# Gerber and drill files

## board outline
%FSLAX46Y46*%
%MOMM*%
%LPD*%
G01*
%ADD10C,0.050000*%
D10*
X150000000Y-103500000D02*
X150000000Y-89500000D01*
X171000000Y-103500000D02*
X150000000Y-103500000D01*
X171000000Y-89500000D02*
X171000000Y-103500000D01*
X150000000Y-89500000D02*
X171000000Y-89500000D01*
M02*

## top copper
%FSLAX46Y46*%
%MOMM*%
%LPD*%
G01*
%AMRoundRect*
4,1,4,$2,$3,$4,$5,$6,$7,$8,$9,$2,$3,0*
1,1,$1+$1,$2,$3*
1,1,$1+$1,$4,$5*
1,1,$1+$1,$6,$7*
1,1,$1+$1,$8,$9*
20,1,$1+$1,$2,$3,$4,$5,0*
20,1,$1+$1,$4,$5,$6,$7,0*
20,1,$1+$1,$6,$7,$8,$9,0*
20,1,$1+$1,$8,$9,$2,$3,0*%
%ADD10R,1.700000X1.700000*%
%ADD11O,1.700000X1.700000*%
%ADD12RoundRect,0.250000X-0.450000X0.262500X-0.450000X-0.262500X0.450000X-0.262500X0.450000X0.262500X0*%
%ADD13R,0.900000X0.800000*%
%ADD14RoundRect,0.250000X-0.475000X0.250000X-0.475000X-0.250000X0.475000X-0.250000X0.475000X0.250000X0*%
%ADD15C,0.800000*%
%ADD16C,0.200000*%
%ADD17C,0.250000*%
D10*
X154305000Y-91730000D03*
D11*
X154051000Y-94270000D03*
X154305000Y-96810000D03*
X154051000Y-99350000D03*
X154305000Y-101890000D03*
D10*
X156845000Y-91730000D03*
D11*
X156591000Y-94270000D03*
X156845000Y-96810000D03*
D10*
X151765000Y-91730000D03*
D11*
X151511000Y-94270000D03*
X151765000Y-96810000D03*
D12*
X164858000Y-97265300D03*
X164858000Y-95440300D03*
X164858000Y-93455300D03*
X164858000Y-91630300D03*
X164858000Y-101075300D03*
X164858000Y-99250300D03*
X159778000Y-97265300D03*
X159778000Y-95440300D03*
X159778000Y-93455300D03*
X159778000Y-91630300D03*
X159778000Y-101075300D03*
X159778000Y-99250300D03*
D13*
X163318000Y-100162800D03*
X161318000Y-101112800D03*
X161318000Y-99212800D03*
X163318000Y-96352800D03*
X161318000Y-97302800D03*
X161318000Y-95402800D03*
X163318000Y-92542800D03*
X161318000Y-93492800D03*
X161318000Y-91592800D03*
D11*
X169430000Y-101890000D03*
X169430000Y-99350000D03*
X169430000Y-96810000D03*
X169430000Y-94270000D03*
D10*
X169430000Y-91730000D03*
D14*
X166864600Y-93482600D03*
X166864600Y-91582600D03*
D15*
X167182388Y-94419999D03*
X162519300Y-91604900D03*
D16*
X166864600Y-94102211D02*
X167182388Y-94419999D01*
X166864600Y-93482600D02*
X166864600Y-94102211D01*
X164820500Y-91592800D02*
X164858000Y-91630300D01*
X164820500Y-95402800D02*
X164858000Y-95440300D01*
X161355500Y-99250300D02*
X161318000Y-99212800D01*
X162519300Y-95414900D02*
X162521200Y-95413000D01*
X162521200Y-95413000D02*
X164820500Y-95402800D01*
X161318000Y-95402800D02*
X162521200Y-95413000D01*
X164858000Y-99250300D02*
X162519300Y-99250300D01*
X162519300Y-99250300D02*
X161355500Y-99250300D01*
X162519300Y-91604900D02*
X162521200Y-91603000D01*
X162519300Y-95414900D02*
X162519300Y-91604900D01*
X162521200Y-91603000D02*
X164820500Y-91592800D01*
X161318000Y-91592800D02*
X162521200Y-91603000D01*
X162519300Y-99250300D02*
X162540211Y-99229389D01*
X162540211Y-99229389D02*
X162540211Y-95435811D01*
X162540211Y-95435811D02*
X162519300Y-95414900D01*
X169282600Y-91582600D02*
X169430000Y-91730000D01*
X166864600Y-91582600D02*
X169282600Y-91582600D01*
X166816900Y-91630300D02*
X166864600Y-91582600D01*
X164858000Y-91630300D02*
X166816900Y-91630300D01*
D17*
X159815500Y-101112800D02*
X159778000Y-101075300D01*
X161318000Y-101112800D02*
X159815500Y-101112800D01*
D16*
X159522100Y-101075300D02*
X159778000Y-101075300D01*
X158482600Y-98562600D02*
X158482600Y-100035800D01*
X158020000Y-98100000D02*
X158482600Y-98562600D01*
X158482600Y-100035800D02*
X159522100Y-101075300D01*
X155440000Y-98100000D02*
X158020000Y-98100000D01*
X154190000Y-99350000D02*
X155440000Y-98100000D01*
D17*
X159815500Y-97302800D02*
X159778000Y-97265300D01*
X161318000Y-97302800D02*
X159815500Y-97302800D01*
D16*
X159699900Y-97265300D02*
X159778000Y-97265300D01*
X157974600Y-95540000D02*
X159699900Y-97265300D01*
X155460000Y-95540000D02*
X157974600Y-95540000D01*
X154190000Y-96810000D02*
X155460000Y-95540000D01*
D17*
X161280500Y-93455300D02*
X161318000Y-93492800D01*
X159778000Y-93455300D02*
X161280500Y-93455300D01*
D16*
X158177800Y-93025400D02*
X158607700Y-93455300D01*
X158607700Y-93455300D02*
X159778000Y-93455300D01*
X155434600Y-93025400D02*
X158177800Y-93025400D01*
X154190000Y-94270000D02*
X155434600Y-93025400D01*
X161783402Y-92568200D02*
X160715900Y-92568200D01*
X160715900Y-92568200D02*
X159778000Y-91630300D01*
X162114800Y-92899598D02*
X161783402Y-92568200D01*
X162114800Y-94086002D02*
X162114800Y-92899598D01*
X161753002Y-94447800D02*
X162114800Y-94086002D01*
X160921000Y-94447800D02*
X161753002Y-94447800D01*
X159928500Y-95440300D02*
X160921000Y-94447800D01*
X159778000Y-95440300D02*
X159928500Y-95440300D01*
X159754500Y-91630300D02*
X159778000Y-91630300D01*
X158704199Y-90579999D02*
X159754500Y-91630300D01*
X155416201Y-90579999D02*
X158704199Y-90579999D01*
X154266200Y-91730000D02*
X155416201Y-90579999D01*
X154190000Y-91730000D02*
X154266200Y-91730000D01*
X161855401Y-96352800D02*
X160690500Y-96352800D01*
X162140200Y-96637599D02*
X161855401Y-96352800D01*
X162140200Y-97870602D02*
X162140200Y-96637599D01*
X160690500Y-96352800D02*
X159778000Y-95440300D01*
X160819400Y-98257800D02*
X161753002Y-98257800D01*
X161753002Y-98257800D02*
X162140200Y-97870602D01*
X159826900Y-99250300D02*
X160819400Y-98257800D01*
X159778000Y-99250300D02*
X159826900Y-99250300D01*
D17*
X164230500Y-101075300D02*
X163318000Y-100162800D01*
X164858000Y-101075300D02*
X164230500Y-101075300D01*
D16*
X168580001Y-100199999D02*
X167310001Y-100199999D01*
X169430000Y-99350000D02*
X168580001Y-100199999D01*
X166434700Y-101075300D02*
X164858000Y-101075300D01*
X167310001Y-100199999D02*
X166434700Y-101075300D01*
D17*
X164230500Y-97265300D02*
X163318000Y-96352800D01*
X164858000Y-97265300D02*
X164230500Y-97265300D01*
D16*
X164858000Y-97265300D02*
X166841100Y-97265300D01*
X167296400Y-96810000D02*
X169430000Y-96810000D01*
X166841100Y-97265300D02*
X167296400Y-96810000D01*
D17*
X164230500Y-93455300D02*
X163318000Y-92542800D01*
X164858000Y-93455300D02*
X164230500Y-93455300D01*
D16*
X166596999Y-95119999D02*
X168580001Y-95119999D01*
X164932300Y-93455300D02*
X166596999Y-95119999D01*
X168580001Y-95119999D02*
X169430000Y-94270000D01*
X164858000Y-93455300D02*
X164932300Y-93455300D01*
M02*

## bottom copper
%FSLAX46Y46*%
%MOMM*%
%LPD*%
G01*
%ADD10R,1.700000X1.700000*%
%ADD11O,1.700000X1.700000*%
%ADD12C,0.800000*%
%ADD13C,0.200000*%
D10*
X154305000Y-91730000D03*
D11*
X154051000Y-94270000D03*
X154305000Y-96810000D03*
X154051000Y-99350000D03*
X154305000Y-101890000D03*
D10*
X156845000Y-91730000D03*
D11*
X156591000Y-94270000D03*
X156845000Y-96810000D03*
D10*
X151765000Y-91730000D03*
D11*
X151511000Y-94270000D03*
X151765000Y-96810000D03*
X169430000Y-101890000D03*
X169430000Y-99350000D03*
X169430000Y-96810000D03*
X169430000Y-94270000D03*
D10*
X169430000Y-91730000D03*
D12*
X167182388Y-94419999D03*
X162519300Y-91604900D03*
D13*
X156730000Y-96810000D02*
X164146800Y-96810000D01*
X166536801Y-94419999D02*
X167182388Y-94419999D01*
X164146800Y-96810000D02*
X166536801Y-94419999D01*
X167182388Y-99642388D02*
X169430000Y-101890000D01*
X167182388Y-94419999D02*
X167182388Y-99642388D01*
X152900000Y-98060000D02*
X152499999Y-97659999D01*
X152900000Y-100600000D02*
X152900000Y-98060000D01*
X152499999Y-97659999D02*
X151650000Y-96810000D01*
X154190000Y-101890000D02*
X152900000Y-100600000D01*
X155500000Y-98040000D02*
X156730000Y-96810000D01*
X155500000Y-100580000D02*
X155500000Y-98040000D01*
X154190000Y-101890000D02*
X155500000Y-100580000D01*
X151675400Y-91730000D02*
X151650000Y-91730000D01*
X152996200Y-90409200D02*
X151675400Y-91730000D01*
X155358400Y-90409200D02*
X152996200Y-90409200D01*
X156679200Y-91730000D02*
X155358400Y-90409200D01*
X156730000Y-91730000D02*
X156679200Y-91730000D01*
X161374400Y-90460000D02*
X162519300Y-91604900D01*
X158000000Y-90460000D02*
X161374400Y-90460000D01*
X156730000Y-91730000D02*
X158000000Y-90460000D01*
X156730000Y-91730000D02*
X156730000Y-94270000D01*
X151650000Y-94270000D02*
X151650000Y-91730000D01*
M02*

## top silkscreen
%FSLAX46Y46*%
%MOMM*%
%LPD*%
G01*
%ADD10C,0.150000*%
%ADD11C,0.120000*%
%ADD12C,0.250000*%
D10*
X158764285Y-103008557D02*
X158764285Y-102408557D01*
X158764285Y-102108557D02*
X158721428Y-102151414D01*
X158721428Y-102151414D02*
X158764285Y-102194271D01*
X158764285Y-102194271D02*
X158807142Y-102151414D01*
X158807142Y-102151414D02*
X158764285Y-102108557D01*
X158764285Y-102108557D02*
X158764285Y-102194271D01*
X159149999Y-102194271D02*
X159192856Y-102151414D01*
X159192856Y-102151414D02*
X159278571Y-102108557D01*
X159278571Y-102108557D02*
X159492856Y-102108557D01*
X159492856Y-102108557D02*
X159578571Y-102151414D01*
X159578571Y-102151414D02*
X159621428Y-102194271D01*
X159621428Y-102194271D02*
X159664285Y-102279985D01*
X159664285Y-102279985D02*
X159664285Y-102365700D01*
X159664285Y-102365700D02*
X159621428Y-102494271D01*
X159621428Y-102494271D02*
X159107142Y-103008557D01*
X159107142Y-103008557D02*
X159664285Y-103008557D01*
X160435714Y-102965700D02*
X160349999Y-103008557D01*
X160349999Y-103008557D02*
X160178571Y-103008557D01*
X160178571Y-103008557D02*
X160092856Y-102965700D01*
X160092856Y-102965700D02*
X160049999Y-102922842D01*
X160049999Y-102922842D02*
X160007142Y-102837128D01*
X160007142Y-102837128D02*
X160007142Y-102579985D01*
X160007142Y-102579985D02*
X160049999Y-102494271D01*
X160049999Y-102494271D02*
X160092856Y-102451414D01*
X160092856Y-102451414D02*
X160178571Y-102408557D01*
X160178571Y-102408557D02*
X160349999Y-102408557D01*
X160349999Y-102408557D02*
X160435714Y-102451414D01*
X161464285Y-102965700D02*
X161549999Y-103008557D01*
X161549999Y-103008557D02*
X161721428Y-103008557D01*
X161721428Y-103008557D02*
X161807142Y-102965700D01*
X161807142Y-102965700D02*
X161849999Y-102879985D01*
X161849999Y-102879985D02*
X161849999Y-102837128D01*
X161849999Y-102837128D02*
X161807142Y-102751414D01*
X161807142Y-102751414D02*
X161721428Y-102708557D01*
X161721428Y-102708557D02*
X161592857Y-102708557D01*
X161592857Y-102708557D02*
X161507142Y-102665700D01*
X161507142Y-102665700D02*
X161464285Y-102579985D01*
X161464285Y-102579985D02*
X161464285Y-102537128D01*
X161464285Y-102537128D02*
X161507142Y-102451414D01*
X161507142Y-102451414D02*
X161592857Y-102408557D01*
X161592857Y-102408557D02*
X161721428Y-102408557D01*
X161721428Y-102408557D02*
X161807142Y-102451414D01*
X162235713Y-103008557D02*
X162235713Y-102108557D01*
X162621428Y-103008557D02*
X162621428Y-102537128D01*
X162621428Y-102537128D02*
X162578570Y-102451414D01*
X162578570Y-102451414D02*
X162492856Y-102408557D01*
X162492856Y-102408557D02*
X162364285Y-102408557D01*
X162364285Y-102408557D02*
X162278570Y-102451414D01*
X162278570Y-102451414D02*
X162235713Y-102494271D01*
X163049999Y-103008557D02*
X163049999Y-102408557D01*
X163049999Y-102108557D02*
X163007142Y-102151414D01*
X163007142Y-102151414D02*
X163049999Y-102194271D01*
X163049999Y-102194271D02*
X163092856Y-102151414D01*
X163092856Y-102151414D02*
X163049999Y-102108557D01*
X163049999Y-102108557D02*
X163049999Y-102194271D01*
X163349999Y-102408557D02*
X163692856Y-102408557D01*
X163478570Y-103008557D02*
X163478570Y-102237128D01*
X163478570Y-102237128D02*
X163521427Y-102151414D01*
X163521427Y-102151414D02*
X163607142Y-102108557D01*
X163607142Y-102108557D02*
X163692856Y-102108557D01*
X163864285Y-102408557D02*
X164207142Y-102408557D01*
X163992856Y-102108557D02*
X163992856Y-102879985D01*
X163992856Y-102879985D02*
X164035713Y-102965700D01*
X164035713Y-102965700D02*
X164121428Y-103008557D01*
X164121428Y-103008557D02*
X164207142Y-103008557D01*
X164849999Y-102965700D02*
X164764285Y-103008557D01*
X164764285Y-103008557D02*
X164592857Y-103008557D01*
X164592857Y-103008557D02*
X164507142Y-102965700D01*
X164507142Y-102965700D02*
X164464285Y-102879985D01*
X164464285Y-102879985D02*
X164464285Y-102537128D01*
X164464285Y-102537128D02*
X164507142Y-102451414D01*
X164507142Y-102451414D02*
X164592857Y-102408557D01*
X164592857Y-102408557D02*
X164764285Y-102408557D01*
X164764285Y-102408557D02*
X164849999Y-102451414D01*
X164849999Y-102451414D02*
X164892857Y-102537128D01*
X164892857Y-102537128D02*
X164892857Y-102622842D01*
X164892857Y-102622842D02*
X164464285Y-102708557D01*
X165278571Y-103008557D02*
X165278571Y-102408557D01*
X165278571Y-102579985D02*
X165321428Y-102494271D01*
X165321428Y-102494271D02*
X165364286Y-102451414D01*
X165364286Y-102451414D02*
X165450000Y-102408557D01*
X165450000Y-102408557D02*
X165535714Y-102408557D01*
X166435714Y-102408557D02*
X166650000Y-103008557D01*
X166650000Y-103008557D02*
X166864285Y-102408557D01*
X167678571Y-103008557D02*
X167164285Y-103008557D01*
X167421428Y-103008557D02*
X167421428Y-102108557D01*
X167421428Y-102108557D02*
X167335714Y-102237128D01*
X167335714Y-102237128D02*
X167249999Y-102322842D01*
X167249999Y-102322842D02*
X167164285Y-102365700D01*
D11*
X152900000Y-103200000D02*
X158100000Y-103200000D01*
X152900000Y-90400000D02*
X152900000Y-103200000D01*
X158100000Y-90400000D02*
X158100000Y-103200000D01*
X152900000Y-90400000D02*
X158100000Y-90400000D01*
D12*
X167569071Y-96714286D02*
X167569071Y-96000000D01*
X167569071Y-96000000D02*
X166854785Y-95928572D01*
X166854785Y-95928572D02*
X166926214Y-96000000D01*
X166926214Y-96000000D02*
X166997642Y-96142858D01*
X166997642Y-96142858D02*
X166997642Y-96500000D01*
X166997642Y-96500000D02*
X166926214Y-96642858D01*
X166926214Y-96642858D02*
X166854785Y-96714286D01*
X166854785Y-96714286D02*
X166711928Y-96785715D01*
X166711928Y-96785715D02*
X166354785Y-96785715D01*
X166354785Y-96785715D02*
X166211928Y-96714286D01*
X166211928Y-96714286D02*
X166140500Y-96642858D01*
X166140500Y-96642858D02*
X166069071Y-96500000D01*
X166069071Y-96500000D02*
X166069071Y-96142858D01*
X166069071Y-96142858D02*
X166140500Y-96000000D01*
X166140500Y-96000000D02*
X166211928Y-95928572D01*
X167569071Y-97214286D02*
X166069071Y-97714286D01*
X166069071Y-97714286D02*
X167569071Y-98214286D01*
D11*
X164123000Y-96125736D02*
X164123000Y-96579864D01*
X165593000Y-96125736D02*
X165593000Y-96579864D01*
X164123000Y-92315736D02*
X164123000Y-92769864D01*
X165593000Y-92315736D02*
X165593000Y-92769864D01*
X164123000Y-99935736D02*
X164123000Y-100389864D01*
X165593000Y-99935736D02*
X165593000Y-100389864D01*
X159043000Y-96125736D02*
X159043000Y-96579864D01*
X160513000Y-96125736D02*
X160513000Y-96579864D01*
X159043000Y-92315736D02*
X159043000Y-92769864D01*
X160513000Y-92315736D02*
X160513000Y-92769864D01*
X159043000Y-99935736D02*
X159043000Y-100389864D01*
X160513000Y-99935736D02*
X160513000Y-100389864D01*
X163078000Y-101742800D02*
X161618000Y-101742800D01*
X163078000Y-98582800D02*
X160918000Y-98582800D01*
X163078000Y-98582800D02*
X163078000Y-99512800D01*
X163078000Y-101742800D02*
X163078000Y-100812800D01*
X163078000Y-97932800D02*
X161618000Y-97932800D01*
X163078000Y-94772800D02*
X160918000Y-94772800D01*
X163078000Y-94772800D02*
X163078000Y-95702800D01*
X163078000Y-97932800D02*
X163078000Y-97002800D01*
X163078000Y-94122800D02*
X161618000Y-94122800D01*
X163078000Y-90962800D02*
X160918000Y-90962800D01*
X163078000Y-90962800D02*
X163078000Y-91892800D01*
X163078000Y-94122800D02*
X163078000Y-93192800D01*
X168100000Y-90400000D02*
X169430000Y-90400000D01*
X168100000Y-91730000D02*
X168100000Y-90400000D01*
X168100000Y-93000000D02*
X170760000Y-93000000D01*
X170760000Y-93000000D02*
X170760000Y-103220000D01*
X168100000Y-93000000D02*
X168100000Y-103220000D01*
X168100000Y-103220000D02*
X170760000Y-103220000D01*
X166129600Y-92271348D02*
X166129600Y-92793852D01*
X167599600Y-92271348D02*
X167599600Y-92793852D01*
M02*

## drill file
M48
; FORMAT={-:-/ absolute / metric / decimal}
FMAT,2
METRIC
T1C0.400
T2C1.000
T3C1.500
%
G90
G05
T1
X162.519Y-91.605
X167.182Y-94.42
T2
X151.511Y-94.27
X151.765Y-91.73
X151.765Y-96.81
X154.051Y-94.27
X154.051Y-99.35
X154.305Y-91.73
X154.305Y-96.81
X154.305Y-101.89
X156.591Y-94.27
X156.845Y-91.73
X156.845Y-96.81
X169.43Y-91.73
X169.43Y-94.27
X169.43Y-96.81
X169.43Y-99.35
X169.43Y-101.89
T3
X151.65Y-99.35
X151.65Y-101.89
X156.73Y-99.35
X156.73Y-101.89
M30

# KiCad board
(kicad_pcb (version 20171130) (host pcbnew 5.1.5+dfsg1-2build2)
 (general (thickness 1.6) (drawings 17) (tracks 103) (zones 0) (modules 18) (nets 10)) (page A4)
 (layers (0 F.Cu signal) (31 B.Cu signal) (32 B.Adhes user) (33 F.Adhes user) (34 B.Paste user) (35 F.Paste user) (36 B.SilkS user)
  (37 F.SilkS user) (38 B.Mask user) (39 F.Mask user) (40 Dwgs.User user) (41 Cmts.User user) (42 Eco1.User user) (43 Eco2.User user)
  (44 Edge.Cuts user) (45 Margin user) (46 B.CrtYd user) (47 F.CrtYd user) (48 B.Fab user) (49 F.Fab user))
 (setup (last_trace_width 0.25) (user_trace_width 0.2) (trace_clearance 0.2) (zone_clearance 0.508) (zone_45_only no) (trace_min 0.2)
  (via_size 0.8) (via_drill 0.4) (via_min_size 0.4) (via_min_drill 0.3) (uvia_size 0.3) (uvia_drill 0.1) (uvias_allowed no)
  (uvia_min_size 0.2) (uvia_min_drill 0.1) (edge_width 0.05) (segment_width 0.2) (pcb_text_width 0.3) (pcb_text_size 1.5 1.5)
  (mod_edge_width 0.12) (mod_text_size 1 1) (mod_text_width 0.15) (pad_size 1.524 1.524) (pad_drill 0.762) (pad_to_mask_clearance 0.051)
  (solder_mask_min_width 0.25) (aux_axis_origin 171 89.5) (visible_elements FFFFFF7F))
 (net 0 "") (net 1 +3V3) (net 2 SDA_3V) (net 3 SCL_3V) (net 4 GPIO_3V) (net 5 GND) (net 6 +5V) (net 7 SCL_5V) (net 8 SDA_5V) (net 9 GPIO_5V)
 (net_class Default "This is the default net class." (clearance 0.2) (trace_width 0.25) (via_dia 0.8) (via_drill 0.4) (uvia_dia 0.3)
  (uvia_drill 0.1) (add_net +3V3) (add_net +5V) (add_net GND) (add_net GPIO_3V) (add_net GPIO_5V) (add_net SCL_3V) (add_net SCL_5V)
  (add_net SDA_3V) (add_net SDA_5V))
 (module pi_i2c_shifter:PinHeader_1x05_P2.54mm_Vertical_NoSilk (layer F.Cu) (at 154.19 91.73)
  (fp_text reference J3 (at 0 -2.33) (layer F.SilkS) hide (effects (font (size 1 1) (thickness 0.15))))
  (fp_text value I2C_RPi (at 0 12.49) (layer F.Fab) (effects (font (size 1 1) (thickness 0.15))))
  (pad 1 thru_hole rect (at 0.115 0) (size 1.7 1.7) (drill 1) (layers *.Cu *.Mask) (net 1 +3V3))
  (pad 2 thru_hole oval (at -0.139 2.54) (size 1.7 1.7) (drill 1) (layers *.Cu *.Mask) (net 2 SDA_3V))
  (pad 3 thru_hole oval (at 0.115 5.08) (size 1.7 1.7) (drill 1) (layers *.Cu *.Mask) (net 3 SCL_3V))
  (pad 4 thru_hole oval (at -0.139 7.62) (size 1.7 1.7) (drill 1) (layers *.Cu *.Mask) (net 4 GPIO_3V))
  (pad 5 thru_hole oval (at 0.115 10.16) (size 1.7 1.7) (drill 1) (layers *.Cu *.Mask) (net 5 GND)))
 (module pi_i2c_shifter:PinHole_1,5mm (layer F.Cu) (at 151.65 99.35)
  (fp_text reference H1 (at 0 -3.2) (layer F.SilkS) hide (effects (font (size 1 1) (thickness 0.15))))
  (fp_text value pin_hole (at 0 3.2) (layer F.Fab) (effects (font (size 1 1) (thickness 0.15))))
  (pad "" np_thru_hole circle (at 0 0) (size 1.5 1.5) (drill 1.5) (layers *.Cu *.Mask)))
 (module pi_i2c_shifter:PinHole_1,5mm (layer F.Cu) (at 151.65 101.89)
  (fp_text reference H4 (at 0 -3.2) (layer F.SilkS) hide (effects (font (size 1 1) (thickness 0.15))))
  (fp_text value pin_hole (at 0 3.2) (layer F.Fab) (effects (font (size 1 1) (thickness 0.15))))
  (pad "" np_thru_hole circle (at 0 0) (size 1.5 1.5) (drill 1.5) (layers *.Cu *.Mask)))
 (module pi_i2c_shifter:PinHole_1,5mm (layer F.Cu) (at 156.73 99.35)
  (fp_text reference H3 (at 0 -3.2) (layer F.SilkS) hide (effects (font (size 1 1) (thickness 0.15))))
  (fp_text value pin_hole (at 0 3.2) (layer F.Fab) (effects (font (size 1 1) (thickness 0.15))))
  (pad "" np_thru_hole circle (at 0 0) (size 1.5 1.5) (drill 1.5) (layers *.Cu *.Mask)))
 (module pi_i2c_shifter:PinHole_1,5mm (layer F.Cu) (at 156.73 101.89)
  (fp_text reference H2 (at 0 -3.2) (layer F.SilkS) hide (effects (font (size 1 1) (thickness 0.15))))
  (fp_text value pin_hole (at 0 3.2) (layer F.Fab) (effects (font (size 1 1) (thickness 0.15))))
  (pad "" np_thru_hole circle (at 0 0) (size 1.5 1.5) (drill 1.5) (layers *.Cu *.Mask)))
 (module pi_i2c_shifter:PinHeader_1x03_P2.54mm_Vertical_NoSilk (layer F.Cu) (at 156.73 91.73)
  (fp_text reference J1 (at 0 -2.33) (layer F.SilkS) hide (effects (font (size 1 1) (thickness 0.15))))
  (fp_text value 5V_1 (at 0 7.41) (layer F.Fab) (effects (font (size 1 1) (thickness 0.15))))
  (pad 1 thru_hole rect (at 0.115 0) (size 1.7 1.7) (drill 1) (layers *.Cu *.Mask) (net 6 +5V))
  (pad 2 thru_hole oval (at -0.139 2.54) (size 1.7 1.7) (drill 1) (layers *.Cu *.Mask) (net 6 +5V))
  (pad 3 thru_hole oval (at 0.115 5.08) (size 1.7 1.7) (drill 1) (layers *.Cu *.Mask) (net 5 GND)))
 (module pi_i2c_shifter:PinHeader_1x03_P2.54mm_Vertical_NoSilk (layer F.Cu) (at 151.65 91.73)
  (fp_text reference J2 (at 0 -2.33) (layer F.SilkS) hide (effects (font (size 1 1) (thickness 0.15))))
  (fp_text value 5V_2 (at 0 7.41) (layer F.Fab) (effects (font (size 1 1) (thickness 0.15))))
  (pad 1 thru_hole rect (at 0.115 0) (size 1.7 1.7) (drill 1) (layers *.Cu *.Mask) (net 6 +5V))
  (pad 2 thru_hole oval (at -0.139 2.54) (size 1.7 1.7) (drill 1) (layers *.Cu *.Mask) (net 6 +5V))
  (pad 3 thru_hole oval (at 0.115 5.08) (size 1.7 1.7) (drill 1) (layers *.Cu *.Mask) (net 5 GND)))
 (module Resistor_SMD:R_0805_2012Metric (layer F.Cu) (at 164.858 96.3528 270)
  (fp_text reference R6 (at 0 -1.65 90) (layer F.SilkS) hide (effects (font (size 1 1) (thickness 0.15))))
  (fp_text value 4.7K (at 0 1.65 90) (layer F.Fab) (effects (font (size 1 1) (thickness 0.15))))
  (fp_line (start -0.227064 0.735) (end 0.227064 0.735) (layer F.SilkS) (width 0.12))
  (fp_line (start -0.227064 -0.735) (end 0.227064 -0.735) (layer F.SilkS) (width 0.12))
  (pad 2 smd roundrect (at 0.9125 0 270) (size 1.025 1.4) (layers F.Cu F.Paste F.Mask) (roundrect_rratio 0.243902) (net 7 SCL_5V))
  (pad 1 smd roundrect (at -0.9125 0 270) (size 1.025 1.4) (layers F.Cu F.Paste F.Mask) (roundrect_rratio 0.243902) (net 6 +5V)))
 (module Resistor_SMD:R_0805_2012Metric (layer F.Cu) (at 164.858 92.5428 270)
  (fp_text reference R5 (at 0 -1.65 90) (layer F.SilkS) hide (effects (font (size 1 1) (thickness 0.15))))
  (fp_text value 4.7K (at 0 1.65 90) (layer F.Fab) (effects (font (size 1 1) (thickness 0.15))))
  (fp_line (start -0.227064 0.735) (end 0.227064 0.735) (layer F.SilkS) (width 0.12))
  (fp_line (start -0.227064 -0.735) (end 0.227064 -0.735) (layer F.SilkS) (width 0.12))
  (pad 2 smd roundrect (at 0.9125 0 270) (size 1.025 1.4) (layers F.Cu F.Paste F.Mask) (roundrect_rratio 0.243902) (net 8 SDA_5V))
  (pad 1 smd roundrect (at -0.9125 0 270) (size 1.025 1.4) (layers F.Cu F.Paste F.Mask) (roundrect_rratio 0.243902) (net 6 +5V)))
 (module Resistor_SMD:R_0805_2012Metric (layer F.Cu) (at 164.858 100.1628 270)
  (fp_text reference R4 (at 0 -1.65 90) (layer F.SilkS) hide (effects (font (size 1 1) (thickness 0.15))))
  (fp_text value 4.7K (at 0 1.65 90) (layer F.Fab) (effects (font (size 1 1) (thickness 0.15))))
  (fp_line (start -0.227064 0.735) (end 0.227064 0.735) (layer F.SilkS) (width 0.12))
  (fp_line (start -0.227064 -0.735) (end 0.227064 -0.735) (layer F.SilkS) (width 0.12))
  (pad 2 smd roundrect (at 0.9125 0 270) (size 1.025 1.4) (layers F.Cu F.Paste F.Mask) (roundrect_rratio 0.243902) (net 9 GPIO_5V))
  (pad 1 smd roundrect (at -0.9125 0 270) (size 1.025 1.4) (layers F.Cu F.Paste F.Mask) (roundrect_rratio 0.243902) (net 6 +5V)))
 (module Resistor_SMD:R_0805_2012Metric (layer F.Cu) (at 159.778 96.3528 270)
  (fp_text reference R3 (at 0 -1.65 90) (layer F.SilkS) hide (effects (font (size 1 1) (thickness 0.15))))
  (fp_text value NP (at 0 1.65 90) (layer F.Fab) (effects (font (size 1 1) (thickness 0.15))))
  (fp_line (start -0.227064 0.735) (end 0.227064 0.735) (layer F.SilkS) (width 0.12))
  (fp_line (start -0.227064 -0.735) (end 0.227064 -0.735) (layer F.SilkS) (width 0.12))
  (pad 2 smd roundrect (at 0.9125 0 270) (size 1.025 1.4) (layers F.Cu F.Paste F.Mask) (roundrect_rratio 0.243902) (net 3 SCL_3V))
  (pad 1 smd roundrect (at -0.9125 0 270) (size 1.025 1.4) (layers F.Cu F.Paste F.Mask) (roundrect_rratio 0.243902) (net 1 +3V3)))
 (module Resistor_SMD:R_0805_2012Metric (layer F.Cu) (at 159.778 92.5428 270)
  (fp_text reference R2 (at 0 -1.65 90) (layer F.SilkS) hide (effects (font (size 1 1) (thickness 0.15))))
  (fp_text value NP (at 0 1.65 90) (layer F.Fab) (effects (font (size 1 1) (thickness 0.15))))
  (fp_line (start -0.227064 0.735) (end 0.227064 0.735) (layer F.SilkS) (width 0.12))
  (fp_line (start -0.227064 -0.735) (end 0.227064 -0.735) (layer F.SilkS) (width 0.12))
  (pad 2 smd roundrect (at 0.9125 0 270) (size 1.025 1.4) (layers F.Cu F.Paste F.Mask) (roundrect_rratio 0.243902) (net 2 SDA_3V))
  (pad 1 smd roundrect (at -0.9125 0 270) (size 1.025 1.4) (layers F.Cu F.Paste F.Mask) (roundrect_rratio 0.243902) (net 1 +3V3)))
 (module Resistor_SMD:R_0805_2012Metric (layer F.Cu) (at 159.778 100.1628 270)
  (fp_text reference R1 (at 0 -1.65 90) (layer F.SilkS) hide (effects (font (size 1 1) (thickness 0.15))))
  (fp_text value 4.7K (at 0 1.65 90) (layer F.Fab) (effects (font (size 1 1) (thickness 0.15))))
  (fp_line (start -0.227064 0.735) (end 0.227064 0.735) (layer F.SilkS) (width 0.12))
  (fp_line (start -0.227064 -0.735) (end 0.227064 -0.735) (layer F.SilkS) (width 0.12))
  (pad 2 smd roundrect (at 0.9125 0 270) (size 1.025 1.4) (layers F.Cu F.Paste F.Mask) (roundrect_rratio 0.243902) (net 4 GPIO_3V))
  (pad 1 smd roundrect (at -0.9125 0 270) (size 1.025 1.4) (layers F.Cu F.Paste F.Mask) (roundrect_rratio 0.243902) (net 1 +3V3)))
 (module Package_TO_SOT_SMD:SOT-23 (layer F.Cu) (at 162.318 100.1628)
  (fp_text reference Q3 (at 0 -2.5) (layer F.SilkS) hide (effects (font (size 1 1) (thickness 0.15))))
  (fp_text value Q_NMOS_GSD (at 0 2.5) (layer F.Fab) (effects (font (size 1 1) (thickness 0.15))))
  (fp_line (start 0.76 1.58) (end -0.7 1.58) (layer F.SilkS) (width 0.12))
  (fp_line (start 0.76 -1.58) (end -1.4 -1.58) (layer F.SilkS) (width 0.12))
  (fp_line (start 0.76 -1.58) (end 0.76 -0.65) (layer F.SilkS) (width 0.12))
  (fp_line (start 0.76 1.58) (end 0.76 0.65) (layer F.SilkS) (width 0.12))
  (pad 3 smd rect (at 1 0) (size 0.9 0.8) (layers F.Cu F.Paste F.Mask) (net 9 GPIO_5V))
  (pad 2 smd rect (at -1 0.95) (size 0.9 0.8) (layers F.Cu F.Paste F.Mask) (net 4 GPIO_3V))
  (pad 1 smd rect (at -1 -0.95) (size 0.9 0.8) (layers F.Cu F.Paste F.Mask) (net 6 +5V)))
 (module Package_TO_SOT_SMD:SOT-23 (layer F.Cu) (at 162.318 96.3528)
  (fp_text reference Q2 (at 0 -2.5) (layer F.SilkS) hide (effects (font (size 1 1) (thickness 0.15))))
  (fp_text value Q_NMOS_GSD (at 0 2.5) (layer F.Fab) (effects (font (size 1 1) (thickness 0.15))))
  (fp_line (start 0.76 1.58) (end -0.7 1.58) (layer F.SilkS) (width 0.12))
  (fp_line (start 0.76 -1.58) (end -1.4 -1.58) (layer F.SilkS) (width 0.12))
  (fp_line (start 0.76 -1.58) (end 0.76 -0.65) (layer F.SilkS) (width 0.12))
  (fp_line (start 0.76 1.58) (end 0.76 0.65) (layer F.SilkS) (width 0.12))
  (pad 3 smd rect (at 1 0) (size 0.9 0.8) (layers F.Cu F.Paste F.Mask) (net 7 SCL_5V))
  (pad 2 smd rect (at -1 0.95) (size 0.9 0.8) (layers F.Cu F.Paste F.Mask) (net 3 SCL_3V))
  (pad 1 smd rect (at -1 -0.95) (size 0.9 0.8) (layers F.Cu F.Paste F.Mask) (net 6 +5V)))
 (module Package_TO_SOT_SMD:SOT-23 (layer F.Cu) (at 162.318 92.5428)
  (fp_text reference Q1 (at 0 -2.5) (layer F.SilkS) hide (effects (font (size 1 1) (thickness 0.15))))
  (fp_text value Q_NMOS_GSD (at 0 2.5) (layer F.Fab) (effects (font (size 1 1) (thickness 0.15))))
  (fp_line (start 0.76 1.58) (end -0.7 1.58) (layer F.SilkS) (width 0.12))
  (fp_line (start 0.76 -1.58) (end -1.4 -1.58) (layer F.SilkS) (width 0.12))
  (fp_line (start 0.76 -1.58) (end 0.76 -0.65) (layer F.SilkS) (width 0.12))
  (fp_line (start 0.76 1.58) (end 0.76 0.65) (layer F.SilkS) (width 0.12))
  (pad 3 smd rect (at 1 0) (size 0.9 0.8) (layers F.Cu F.Paste F.Mask) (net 8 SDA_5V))
  (pad 2 smd rect (at -1 0.95) (size 0.9 0.8) (layers F.Cu F.Paste F.Mask) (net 2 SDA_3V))
  (pad 1 smd rect (at -1 -0.95) (size 0.9 0.8) (layers F.Cu F.Paste F.Mask) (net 6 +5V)))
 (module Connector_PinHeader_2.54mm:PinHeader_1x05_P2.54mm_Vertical (layer F.Cu) (at 169.43 91.73)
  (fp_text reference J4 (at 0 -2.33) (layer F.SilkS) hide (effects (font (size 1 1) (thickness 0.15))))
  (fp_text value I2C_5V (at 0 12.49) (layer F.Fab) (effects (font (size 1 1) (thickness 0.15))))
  (fp_line (start -1.33 -1.33) (end 0 -1.33) (layer F.SilkS) (width 0.12))
  (fp_line (start -1.33 0) (end -1.33 -1.33) (layer F.SilkS) (width 0.12))
  (fp_line (start -1.33 1.27) (end 1.33 1.27) (layer F.SilkS) (width 0.12))
  (fp_line (start 1.33 1.27) (end 1.33 11.49) (layer F.SilkS) (width 0.12))
  (fp_line (start -1.33 1.27) (end -1.33 11.49) (layer F.SilkS) (width 0.12))
  (fp_line (start -1.33 11.49) (end 1.33 11.49) (layer F.SilkS) (width 0.12))
  (pad 5 thru_hole oval (at 0 10.16) (size 1.7 1.7) (drill 1) (layers *.Cu *.Mask) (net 5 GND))
  (pad 4 thru_hole oval (at 0 7.62) (size 1.7 1.7) (drill 1) (layers *.Cu *.Mask) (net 9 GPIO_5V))
  (pad 3 thru_hole oval (at 0 5.08) (size 1.7 1.7) (drill 1) (layers *.Cu *.Mask) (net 7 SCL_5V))
  (pad 2 thru_hole oval (at 0 2.54) (size 1.7 1.7) (drill 1) (layers *.Cu *.Mask) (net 8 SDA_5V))
  (pad 1 thru_hole rect (at 0 0) (size 1.7 1.7) (drill 1) (layers *.Cu *.Mask) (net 6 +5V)))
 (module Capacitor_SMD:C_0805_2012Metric (layer F.Cu) (at 166.8646 92.5326 270)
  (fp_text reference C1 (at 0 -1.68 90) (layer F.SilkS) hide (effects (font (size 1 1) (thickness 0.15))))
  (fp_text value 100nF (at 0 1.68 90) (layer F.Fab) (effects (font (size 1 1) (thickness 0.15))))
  (fp_line (start -0.261252 0.735) (end 0.261252 0.735) (layer F.SilkS) (width 0.12))
  (fp_line (start -0.261252 -0.735) (end 0.261252 -0.735) (layer F.SilkS) (width 0.12))
  (pad 2 smd roundrect (at 0.95 0 270) (size 1 1.45) (layers F.Cu F.Paste F.Mask) (roundrect_rratio 0.25) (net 5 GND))
  (pad 1 smd roundrect (at -0.95 0 270) (size 1 1.45) (layers F.Cu F.Paste F.Mask) (roundrect_rratio 0.25) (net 6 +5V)))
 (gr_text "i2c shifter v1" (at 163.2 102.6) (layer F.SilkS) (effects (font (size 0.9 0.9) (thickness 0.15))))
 (gr_line (start 152.9 103.2) (end 158.1 103.2) (layer F.SilkS) (width 0.12))
 (gr_line (start 152.9 90.4) (end 152.9 103.2) (layer F.SilkS) (width 0.12))
 (gr_line (start 158.1 90.4) (end 158.1 103.2) (layer F.SilkS) (width 0.12))
 (gr_line (start 152.9 90.4) (end 158.1 90.4) (layer F.SilkS) (width 0.12))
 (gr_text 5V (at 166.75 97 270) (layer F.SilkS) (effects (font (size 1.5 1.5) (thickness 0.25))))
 (gr_line (start 150 103.5) (end 150 89.5) (layer Edge.Cuts) (width 0.05))
 (gr_line (start 171 103.5) (end 150 103.5) (layer Edge.Cuts) (width 0.05))
 (gr_line (start 171 89.5) (end 171 103.5) (layer Edge.Cuts) (width 0.05))
 (gr_line (start 150 89.5) (end 171 89.5) (layer Edge.Cuts) (width 0.05))
 (via (at 167.182388 94.419999) (size 0.8) (drill 0.4) (layers F.Cu B.Cu) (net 5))
 (segment (start 166.8646 94.102211) (end 167.182388 94.419999) (width 0.2) (layer F.Cu) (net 5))
 (segment (start 166.8646 93.4826) (end 166.8646 94.102211) (width 0.2) (layer F.Cu) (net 5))
 (segment (start 156.73 96.81) (end 164.1468 96.81) (width 0.2) (layer B.Cu) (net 5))
 (segment (start 166.536801 94.419999) (end 167.182388 94.419999) (width 0.2) (layer B.Cu) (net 5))
 (segment (start 164.1468 96.81) (end 166.536801 94.419999) (width 0.2) (layer B.Cu) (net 5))
 (segment (start 167.182388 99.642388) (end 169.43 101.89) (width 0.2) (layer B.Cu) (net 5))
 (segment (start 167.182388 94.419999) (end 167.182388 99.642388) (width 0.2) (layer B.Cu) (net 5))
 (segment (start 152.9 98.06) (end 152.499999 97.659999) (width 0.2) (layer B.Cu) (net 5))
 (segment (start 152.9 100.6) (end 152.9 98.06) (width 0.2) (layer B.Cu) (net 5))
 (segment (start 152.499999 97.659999) (end 151.65 96.81) (width 0.2) (layer B.Cu) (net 5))
 (segment (start 154.19 101.89) (end 152.9 100.6) (width 0.2) (layer B.Cu) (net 5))
 (segment (start 155.5 98.04) (end 156.73 96.81) (width 0.2) (layer B.Cu) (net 5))
 (segment (start 155.5 100.58) (end 155.5 98.04) (width 0.2) (layer B.Cu) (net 5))
 (segment (start 154.19 101.89) (end 155.5 100.58) (width 0.2) (layer B.Cu) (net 5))
 (segment (start 164.8205 91.5928) (end 164.858 91.6303) (width 0.2) (layer F.Cu) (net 6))
 (segment (start 164.8205 95.4028) (end 164.858 95.4403) (width 0.2) (layer F.Cu) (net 6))
 (segment (start 161.3555 99.2503) (end 161.318 99.2128) (width 0.2) (layer F.Cu) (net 6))
 (segment (start 162.5193 95.4149) (end 162.5212 95.413) (width 0.2) (layer F.Cu) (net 6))
 (segment (start 162.5212 95.413) (end 164.8205 95.4028) (width 0.2) (layer F.Cu) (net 6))
 (segment (start 161.318 95.4028) (end 162.5212 95.413) (width 0.2) (layer F.Cu) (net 6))
 (segment (start 164.858 99.2503) (end 162.5193 99.2503) (width 0.2) (layer F.Cu) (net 6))
 (segment (start 162.5193 99.2503) (end 161.3555 99.2503) (width 0.2) (layer F.Cu) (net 6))
 (segment (start 162.5193 91.6049) (end 162.5212 91.603) (width 0.2) (layer F.Cu) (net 6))
 (segment (start 162.5193 95.4149) (end 162.5193 91.6049) (width 0.2) (layer F.Cu) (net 6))
 (segment (start 162.5212 91.603) (end 164.8205 91.5928) (width 0.2) (layer F.Cu) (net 6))
 (segment (start 161.318 91.5928) (end 162.5212 91.603) (width 0.2) (layer F.Cu) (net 6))
 (segment (start 162.5193 99.2503) (end 162.540211 99.229389) (width 0.2) (layer F.Cu) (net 6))
 (segment (start 162.540211 99.229389) (end 162.540211 95.435811) (width 0.2) (layer F.Cu) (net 6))
 (segment (start 162.540211 95.435811) (end 162.5193 95.4149) (width 0.2) (layer F.Cu) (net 6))
 (segment (start 169.2826 91.5826) (end 169.43 91.73) (width 0.2) (layer F.Cu) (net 6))
 (segment (start 166.8646 91.5826) (end 169.2826 91.5826) (width 0.2) (layer F.Cu) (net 6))
 (segment (start 166.8169 91.6303) (end 166.8646 91.5826) (width 0.2) (layer F.Cu) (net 6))
 (segment (start 164.858 91.6303) (end 166.8169 91.6303) (width 0.2) (layer F.Cu) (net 6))
 (segment (start 151.6754 91.73) (end 151.65 91.73) (width 0.2) (layer B.Cu) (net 6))
 (segment (start 152.9962 90.4092) (end 151.6754 91.73) (width 0.2) (layer B.Cu) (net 6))
 (segment (start 155.3584 90.4092) (end 152.9962 90.4092) (width 0.2) (layer B.Cu) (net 6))
 (segment (start 156.6792 91.73) (end 155.3584 90.4092) (width 0.2) (layer B.Cu) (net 6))
 (segment (start 156.73 91.73) (end 156.6792 91.73) (width 0.2) (layer B.Cu) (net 6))
 (via (at 162.5193 91.6049) (size 0.8) (drill 0.4) (layers F.Cu B.Cu) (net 6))
 (segment (start 161.3744 90.46) (end 162.5193 91.6049) (width 0.2) (layer B.Cu) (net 6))
 (segment (start 158 90.46) (end 161.3744 90.46) (width 0.2) (layer B.Cu) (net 6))
 (segment (start 156.73 91.73) (end 158 90.46) (width 0.2) (layer B.Cu) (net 6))
 (segment (start 156.73 91.73) (end 156.73 94.27) (width 0.2) (layer B.Cu) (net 6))
 (segment (start 151.65 94.27) (end 151.65 91.73) (width 0.2) (layer B.Cu) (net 6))
 (segment (start 159.8155 101.1128) (end 159.778 101.0753) (width 0.25) (layer F.Cu) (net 4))
 (segment (start 161.318 101.1128) (end 159.8155 101.1128) (width 0.25) (layer F.Cu) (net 4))
 (segment (start 159.5221 101.0753) (end 159.778 101.0753) (width 0.2) (layer F.Cu) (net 4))
 (segment (start 158.4826 98.5626) (end 158.4826 100.0358) (width 0.2) (layer F.Cu) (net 4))
 (segment (start 158.02 98.1) (end 158.4826 98.5626) (width 0.2) (layer F.Cu) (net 4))
 (segment (start 158.4826 100.0358) (end 159.5221 101.0753) (width 0.2) (layer F.Cu) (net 4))
 (segment (start 155.44 98.1) (end 158.02 98.1) (width 0.2) (layer F.Cu) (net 4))
 (segment (start 154.19 99.35) (end 155.44 98.1) (width 0.2) (layer F.Cu) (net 4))
 (segment (start 159.8155 97.3028) (end 159.778 97.2653) (width 0.25) (layer F.Cu) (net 3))
 (segment (start 161.318 97.3028) (end 159.8155 97.3028) (width 0.25) (layer F.Cu) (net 3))
 (segment (start 159.6999 97.2653) (end 159.778 97.2653) (width 0.2) (layer F.Cu) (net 3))
 (segment (start 157.9746 95.54) (end 159.6999 97.2653) (width 0.2) (layer F.Cu) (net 3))
 (segment (start 155.46 95.54) (end 157.9746 95.54) (width 0.2) (layer F.Cu) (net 3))
 (segment (start 154.19 96.81) (end 155.46 95.54) (width 0.2) (layer F.Cu) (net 3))
 (segment (start 161.2805 93.4553) (end 161.318 93.4928) (width 0.25) (layer F.Cu) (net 2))
 (segment (start 159.778 93.4553) (end 161.2805 93.4553) (width 0.25) (layer F.Cu) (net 2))
 (segment (start 158.1778 93.0254) (end 158.6077 93.4553) (width 0.2) (layer F.Cu) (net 2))
 (segment (start 158.6077 93.4553) (end 159.778 93.4553) (width 0.2) (layer F.Cu) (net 2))
 (segment (start 155.4346 93.0254) (end 158.1778 93.0254) (width 0.2) (layer F.Cu) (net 2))
 (segment (start 154.19 94.27) (end 155.4346 93.0254) (width 0.2) (layer F.Cu) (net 2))
 (segment (start 161.783402 92.5682) (end 160.7159 92.5682) (width 0.2) (layer F.Cu) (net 1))
 (segment (start 160.7159 92.5682) (end 159.778 91.6303) (width 0.2) (layer F.Cu) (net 1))
 (segment (start 162.1148 92.899598) (end 161.783402 92.5682) (width 0.2) (layer F.Cu) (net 1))
 (segment (start 162.1148 94.086002) (end 162.1148 92.899598) (width 0.2) (layer F.Cu) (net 1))
 (segment (start 161.753002 94.4478) (end 162.1148 94.086002) (width 0.2) (layer F.Cu) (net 1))
 (segment (start 160.921 94.4478) (end 161.753002 94.4478) (width 0.2) (layer F.Cu) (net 1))
 (segment (start 159.9285 95.4403) (end 160.921 94.4478) (width 0.2) (layer F.Cu) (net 1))
 (segment (start 159.778 95.4403) (end 159.9285 95.4403) (width 0.2) (layer F.Cu) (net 1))
 (segment (start 159.7545 91.6303) (end 159.778 91.6303) (width 0.2) (layer F.Cu) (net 1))
 (segment (start 158.704199 90.579999) (end 159.7545 91.6303) (width 0.2) (layer F.Cu) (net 1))
 (segment (start 155.416201 90.579999) (end 158.704199 90.579999) (width 0.2) (layer F.Cu) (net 1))
 (segment (start 154.2662 91.73) (end 155.416201 90.579999) (width 0.2) (layer F.Cu) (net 1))
 (segment (start 154.19 91.73) (end 154.2662 91.73) (width 0.2) (layer F.Cu) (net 1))
 (segment (start 161.855401 96.3528) (end 160.6905 96.3528) (width 0.2) (layer F.Cu) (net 1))
 (segment (start 162.1402 96.637599) (end 161.855401 96.3528) (width 0.2) (layer F.Cu) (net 1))
 (segment (start 162.1402 97.870602) (end 162.1402 96.637599) (width 0.2) (layer F.Cu) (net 1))
 (segment (start 160.6905 96.3528) (end 159.778 95.4403) (width 0.2) (layer F.Cu) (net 1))
 (segment (start 160.8194 98.2578) (end 161.753002 98.2578) (width 0.2) (layer F.Cu) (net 1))
 (segment (start 161.753002 98.2578) (end 162.1402 97.870602) (width 0.2) (layer F.Cu) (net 1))
 (segment (start 159.8269 99.2503) (end 160.8194 98.2578) (width 0.2) (layer F.Cu) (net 1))
 (segment (start 159.778 99.2503) (end 159.8269 99.2503) (width 0.2) (layer F.Cu) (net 1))
 (segment (start 164.2305 101.0753) (end 163.318 100.1628) (width 0.25) (layer F.Cu) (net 9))
 (segment (start 164.858 101.0753) (end 164.2305 101.0753) (width 0.25) (layer F.Cu) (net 9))
 (segment (start 168.580001 100.199999) (end 167.310001 100.199999) (width 0.2) (layer F.Cu) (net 9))
 (segment (start 169.43 99.35) (end 168.580001 100.199999) (width 0.2) (layer F.Cu) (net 9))
 (segment (start 166.4347 101.0753) (end 164.858 101.0753) (width 0.2) (layer F.Cu) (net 9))
 (segment (start 167.310001 100.199999) (end 166.4347 101.0753) (width 0.2) (layer F.Cu) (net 9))
 (segment (start 164.2305 97.2653) (end 163.318 96.3528) (width 0.25) (layer F.Cu) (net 7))
 (segment (start 164.858 97.2653) (end 164.2305 97.2653) (width 0.25) (layer F.Cu) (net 7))
 (segment (start 164.858 97.2653) (end 166.8411 97.2653) (width 0.2) (layer F.Cu) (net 7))
 (segment (start 167.2964 96.81) (end 169.43 96.81) (width 0.2) (layer F.Cu) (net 7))
 (segment (start 166.8411 97.2653) (end 167.2964 96.81) (width 0.2) (layer F.Cu) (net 7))
 (segment (start 164.2305 93.4553) (end 163.318 92.5428) (width 0.25) (layer F.Cu) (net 8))
 (segment (start 164.858 93.4553) (end 164.2305 93.4553) (width 0.25) (layer F.Cu) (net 8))
 (segment (start 166.596999 95.119999) (end 168.580001 95.119999) (width 0.2) (layer F.Cu) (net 8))
 (segment (start 164.9323 93.4553) (end 166.596999 95.119999) (width 0.2) (layer F.Cu) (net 8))
 (segment (start 168.580001 95.119999) (end 169.43 94.27) (width 0.2) (layer F.Cu) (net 8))
 (segment (start 164.858 93.4553) (end 164.9323 93.4553) (width 0.2) (layer F.Cu) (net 8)))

